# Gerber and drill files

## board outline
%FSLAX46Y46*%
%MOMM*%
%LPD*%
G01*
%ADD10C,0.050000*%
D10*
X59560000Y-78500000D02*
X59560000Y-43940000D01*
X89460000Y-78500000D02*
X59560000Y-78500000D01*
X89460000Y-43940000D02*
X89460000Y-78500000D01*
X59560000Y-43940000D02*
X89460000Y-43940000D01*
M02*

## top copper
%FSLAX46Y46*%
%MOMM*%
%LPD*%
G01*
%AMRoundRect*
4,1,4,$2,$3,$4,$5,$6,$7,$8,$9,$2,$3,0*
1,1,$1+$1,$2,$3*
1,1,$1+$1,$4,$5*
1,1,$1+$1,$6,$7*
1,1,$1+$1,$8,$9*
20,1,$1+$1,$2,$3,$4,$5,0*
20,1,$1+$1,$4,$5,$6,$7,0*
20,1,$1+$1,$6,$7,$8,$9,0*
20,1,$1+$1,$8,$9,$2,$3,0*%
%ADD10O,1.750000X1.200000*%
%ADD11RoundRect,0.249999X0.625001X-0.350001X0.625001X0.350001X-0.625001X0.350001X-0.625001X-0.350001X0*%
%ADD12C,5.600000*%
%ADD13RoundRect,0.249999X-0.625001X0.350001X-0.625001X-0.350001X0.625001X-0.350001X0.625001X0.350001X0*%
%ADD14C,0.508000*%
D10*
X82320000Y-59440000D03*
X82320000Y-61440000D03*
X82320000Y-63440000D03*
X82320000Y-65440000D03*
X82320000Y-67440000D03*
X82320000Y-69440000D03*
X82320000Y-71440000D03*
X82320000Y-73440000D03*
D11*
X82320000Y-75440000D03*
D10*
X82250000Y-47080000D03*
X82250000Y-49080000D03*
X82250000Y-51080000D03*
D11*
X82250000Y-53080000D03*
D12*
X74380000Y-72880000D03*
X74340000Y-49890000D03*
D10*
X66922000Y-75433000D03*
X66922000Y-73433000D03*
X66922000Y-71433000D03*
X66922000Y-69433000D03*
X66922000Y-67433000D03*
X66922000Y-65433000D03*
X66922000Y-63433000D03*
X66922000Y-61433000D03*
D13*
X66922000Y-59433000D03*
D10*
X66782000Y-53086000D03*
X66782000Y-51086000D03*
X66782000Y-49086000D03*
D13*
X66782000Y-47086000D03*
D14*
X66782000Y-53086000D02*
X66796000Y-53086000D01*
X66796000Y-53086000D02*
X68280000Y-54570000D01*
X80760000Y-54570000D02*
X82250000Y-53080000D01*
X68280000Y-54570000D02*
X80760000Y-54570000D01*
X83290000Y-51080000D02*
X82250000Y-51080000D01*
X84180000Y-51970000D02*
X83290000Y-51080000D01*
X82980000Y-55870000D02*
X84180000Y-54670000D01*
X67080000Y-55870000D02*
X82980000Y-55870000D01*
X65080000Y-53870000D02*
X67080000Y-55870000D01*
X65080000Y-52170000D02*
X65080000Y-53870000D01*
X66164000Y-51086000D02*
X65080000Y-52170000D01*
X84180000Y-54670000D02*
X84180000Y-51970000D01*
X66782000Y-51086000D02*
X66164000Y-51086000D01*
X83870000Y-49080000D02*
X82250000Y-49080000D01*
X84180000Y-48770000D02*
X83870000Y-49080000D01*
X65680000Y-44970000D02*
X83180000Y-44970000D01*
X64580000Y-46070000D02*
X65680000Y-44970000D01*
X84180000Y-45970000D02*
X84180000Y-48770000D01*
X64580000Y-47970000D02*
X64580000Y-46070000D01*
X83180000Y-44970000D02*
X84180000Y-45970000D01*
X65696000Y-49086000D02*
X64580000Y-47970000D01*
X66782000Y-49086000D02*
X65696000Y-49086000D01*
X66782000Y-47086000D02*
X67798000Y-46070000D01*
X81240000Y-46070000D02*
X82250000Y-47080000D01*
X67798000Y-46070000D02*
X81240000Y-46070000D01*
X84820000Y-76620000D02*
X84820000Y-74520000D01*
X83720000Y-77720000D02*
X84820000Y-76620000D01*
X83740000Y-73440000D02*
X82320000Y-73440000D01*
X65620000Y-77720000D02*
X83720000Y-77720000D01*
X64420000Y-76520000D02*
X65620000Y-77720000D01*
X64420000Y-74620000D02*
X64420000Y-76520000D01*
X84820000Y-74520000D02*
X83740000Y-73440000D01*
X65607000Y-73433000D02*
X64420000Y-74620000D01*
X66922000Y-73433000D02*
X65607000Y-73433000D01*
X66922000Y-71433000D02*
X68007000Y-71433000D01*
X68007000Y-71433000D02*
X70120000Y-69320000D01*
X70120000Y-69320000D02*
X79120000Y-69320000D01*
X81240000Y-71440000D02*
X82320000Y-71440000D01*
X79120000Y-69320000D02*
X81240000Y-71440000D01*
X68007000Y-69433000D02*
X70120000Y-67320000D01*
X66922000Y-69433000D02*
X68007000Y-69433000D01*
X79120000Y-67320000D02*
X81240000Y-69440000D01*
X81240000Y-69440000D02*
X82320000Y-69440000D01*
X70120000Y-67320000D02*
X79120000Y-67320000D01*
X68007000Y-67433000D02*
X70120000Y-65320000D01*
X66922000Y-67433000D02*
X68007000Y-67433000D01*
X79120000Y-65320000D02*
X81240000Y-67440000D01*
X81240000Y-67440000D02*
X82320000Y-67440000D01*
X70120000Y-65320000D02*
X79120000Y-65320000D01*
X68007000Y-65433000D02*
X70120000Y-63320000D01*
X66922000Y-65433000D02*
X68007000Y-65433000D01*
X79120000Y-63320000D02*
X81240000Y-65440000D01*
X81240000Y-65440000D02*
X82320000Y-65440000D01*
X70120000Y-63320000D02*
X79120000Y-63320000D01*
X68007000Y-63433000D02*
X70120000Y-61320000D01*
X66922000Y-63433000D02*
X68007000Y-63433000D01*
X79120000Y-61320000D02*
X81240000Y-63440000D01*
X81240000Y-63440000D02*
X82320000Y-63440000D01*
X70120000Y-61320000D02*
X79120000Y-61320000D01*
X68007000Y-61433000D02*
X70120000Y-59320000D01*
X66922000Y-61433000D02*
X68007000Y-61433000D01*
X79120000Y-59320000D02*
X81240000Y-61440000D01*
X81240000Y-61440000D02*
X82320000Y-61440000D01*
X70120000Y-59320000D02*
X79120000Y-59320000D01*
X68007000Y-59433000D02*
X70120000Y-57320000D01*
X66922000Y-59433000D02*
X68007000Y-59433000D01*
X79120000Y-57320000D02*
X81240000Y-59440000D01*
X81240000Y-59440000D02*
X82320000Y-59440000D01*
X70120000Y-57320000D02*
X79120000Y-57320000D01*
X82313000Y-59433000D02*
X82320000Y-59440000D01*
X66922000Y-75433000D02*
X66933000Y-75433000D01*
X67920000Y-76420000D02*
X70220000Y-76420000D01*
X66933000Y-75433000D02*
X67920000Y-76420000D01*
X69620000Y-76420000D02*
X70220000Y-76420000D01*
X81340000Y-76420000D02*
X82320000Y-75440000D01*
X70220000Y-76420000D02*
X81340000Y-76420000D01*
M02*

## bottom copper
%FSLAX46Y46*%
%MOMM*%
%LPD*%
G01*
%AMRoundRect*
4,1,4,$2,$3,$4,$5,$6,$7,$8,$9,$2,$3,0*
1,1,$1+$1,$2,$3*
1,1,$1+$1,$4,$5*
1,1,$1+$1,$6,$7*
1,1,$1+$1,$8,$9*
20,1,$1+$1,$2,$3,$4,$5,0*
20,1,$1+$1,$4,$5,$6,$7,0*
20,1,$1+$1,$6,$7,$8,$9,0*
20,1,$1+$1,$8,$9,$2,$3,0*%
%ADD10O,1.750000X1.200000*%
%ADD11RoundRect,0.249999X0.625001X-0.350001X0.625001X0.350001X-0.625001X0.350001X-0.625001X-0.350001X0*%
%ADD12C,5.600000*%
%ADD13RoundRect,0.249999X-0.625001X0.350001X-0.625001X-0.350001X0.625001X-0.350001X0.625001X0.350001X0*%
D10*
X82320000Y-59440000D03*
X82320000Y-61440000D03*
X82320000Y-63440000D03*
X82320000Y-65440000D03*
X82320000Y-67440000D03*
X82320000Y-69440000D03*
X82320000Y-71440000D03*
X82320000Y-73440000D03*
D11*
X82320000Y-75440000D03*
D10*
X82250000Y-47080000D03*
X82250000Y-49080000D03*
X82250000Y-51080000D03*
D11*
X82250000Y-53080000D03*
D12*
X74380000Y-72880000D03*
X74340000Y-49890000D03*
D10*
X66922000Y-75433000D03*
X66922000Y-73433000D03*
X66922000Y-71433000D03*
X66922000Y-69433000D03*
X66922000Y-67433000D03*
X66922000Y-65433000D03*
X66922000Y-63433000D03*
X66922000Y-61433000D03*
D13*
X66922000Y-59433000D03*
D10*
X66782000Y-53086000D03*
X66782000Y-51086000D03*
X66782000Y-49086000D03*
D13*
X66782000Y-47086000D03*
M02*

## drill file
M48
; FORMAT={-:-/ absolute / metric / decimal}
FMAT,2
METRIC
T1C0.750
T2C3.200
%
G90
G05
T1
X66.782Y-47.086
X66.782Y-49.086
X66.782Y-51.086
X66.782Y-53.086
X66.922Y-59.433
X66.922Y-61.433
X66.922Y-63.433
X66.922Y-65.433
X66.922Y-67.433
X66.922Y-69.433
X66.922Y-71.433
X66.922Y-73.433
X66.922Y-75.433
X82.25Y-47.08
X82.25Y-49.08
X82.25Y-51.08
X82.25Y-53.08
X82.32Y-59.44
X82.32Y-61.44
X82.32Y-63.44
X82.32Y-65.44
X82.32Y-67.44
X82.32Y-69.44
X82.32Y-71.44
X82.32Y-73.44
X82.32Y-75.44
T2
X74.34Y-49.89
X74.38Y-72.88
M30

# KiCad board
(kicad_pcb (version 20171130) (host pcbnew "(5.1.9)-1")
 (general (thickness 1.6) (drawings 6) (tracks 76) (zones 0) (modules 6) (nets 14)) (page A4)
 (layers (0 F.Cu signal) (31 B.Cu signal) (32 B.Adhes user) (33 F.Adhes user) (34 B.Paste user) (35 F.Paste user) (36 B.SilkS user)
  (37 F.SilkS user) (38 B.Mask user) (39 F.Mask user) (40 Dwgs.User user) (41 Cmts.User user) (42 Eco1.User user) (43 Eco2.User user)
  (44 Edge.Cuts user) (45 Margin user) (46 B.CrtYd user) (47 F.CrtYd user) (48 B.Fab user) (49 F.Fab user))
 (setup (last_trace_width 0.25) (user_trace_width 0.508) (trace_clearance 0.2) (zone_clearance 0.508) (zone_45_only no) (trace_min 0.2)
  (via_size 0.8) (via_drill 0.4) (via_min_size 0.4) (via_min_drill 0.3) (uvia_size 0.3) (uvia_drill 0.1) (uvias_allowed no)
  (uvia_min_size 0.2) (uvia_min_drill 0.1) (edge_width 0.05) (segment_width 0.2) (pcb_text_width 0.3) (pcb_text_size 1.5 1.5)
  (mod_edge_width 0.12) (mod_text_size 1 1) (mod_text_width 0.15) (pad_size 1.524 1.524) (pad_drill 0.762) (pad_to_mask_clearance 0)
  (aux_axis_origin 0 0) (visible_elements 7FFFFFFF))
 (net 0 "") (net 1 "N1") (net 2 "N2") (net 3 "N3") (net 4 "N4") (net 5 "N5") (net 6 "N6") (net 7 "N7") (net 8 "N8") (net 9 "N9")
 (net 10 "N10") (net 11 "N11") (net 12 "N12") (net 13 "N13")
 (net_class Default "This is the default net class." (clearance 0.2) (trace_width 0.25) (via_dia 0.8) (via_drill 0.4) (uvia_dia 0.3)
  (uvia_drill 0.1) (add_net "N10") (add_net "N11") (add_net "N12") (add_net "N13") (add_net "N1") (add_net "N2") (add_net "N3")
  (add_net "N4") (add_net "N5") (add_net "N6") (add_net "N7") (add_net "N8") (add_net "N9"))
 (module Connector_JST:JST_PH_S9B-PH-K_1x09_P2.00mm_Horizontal (layer F.Cu) (at 82.32 75.44 90)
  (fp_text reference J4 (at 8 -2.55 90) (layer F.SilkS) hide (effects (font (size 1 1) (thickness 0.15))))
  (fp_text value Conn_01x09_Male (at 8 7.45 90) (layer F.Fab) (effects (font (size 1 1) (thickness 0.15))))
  (pad 9 thru_hole oval (at 16 0 90) (size 1.2 1.75) (drill 0.75) (layers *.Cu *.Mask) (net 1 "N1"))
  (pad 8 thru_hole oval (at 14 0 90) (size 1.2 1.75) (drill 0.75) (layers *.Cu *.Mask) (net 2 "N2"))
  (pad 7 thru_hole oval (at 12 0 90) (size 1.2 1.75) (drill 0.75) (layers *.Cu *.Mask) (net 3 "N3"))
  (pad 6 thru_hole oval (at 10 0 90) (size 1.2 1.75) (drill 0.75) (layers *.Cu *.Mask) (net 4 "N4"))
  (pad 5 thru_hole oval (at 8 0 90) (size 1.2 1.75) (drill 0.75) (layers *.Cu *.Mask) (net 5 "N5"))
  (pad 4 thru_hole oval (at 6 0 90) (size 1.2 1.75) (drill 0.75) (layers *.Cu *.Mask) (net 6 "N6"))
  (pad 3 thru_hole oval (at 4 0 90) (size 1.2 1.75) (drill 0.75) (layers *.Cu *.Mask) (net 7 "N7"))
  (pad 2 thru_hole oval (at 2 0 90) (size 1.2 1.75) (drill 0.75) (layers *.Cu *.Mask) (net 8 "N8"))
  (pad 1 thru_hole roundrect (at 0 0 90) (size 1.2 1.75) (drill 0.75) (layers *.Cu *.Mask) (roundrect_rratio 0.2083325) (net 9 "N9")))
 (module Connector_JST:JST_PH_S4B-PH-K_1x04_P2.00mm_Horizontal (layer F.Cu) (at 82.25 53.08 90)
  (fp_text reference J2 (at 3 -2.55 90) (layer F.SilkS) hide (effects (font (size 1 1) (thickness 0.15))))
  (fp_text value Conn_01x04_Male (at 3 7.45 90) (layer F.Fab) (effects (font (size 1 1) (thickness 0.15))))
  (pad 4 thru_hole oval (at 6 0 90) (size 1.2 1.75) (drill 0.75) (layers *.Cu *.Mask) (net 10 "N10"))
  (pad 3 thru_hole oval (at 4 0 90) (size 1.2 1.75) (drill 0.75) (layers *.Cu *.Mask) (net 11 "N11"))
  (pad 2 thru_hole oval (at 2 0 90) (size 1.2 1.75) (drill 0.75) (layers *.Cu *.Mask) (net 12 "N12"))
  (pad 1 thru_hole roundrect (at 0 0 90) (size 1.2 1.75) (drill 0.75) (layers *.Cu *.Mask) (roundrect_rratio 0.2083325) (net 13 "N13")))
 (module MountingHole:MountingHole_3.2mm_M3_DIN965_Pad (layer F.Cu) (at 74.38 72.88)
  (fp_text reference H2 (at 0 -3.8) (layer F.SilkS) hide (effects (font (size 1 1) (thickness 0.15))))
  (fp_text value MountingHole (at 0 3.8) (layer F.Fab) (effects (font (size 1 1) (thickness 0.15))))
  (pad 1 thru_hole circle (at 0 0) (size 5.6 5.6) (drill 3.2) (layers *.Cu *.Mask)))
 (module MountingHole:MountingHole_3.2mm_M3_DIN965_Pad (layer F.Cu) (at 74.34 49.89)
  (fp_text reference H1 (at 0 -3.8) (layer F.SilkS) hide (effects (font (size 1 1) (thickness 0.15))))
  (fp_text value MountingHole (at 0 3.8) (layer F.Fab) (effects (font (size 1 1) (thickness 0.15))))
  (pad 1 thru_hole circle (at 0 0) (size 5.6 5.6) (drill 3.2) (layers *.Cu *.Mask)))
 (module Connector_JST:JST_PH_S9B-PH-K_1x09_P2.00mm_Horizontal (layer F.Cu) (at 66.922 59.433 270)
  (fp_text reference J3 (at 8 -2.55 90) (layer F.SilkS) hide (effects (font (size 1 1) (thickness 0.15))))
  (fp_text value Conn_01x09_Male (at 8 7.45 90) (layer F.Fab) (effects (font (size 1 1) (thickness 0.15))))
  (pad 9 thru_hole oval (at 16 0 270) (size 1.2 1.75) (drill 0.75) (layers *.Cu *.Mask) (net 9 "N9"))
  (pad 8 thru_hole oval (at 14 0 270) (size 1.2 1.75) (drill 0.75) (layers *.Cu *.Mask) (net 8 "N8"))
  (pad 7 thru_hole oval (at 12 0 270) (size 1.2 1.75) (drill 0.75) (layers *.Cu *.Mask) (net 7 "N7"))
  (pad 6 thru_hole oval (at 10 0 270) (size 1.2 1.75) (drill 0.75) (layers *.Cu *.Mask) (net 6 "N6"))
  (pad 5 thru_hole oval (at 8 0 270) (size 1.2 1.75) (drill 0.75) (layers *.Cu *.Mask) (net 5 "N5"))
  (pad 4 thru_hole oval (at 6 0 270) (size 1.2 1.75) (drill 0.75) (layers *.Cu *.Mask) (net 4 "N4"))
  (pad 3 thru_hole oval (at 4 0 270) (size 1.2 1.75) (drill 0.75) (layers *.Cu *.Mask) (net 3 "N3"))
  (pad 2 thru_hole oval (at 2 0 270) (size 1.2 1.75) (drill 0.75) (layers *.Cu *.Mask) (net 2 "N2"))
  (pad 1 thru_hole roundrect (at 0 0 270) (size 1.2 1.75) (drill 0.75) (layers *.Cu *.Mask) (roundrect_rratio 0.2083325) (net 1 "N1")))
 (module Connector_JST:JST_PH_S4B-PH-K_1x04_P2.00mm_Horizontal (layer F.Cu) (at 66.782 47.086 270)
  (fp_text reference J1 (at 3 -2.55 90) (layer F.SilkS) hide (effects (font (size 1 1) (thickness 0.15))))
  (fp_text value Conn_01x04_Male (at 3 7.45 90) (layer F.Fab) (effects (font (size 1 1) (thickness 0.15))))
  (pad 4 thru_hole oval (at 6 0 270) (size 1.2 1.75) (drill 0.75) (layers *.Cu *.Mask) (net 13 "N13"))
  (pad 3 thru_hole oval (at 4 0 270) (size 1.2 1.75) (drill 0.75) (layers *.Cu *.Mask) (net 12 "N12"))
  (pad 2 thru_hole oval (at 2 0 270) (size 1.2 1.75) (drill 0.75) (layers *.Cu *.Mask) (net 11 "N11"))
  (pad 1 thru_hole roundrect (at 0 0 270) (size 1.2 1.75) (drill 0.75) (layers *.Cu *.Mask) (roundrect_rratio 0.2083325) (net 10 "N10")))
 (gr_line (start 59.56 78.5) (end 59.56 43.94) (layer Edge.Cuts) (width 0.05))
 (gr_line (start 89.46 78.5) (end 59.56 78.5) (layer Edge.Cuts) (width 0.05))
 (gr_line (start 89.46 43.94) (end 89.46 78.5) (layer Edge.Cuts) (width 0.05))
 (gr_line (start 59.56 43.94) (end 89.46 43.94) (layer Edge.Cuts) (width 0.05))
 (segment (start 66.782 53.086) (end 66.796 53.086) (width 0.508) (layer F.Cu) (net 13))
 (segment (start 66.796 53.086) (end 68.28 54.57) (width 0.508) (layer F.Cu) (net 13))
 (segment (start 80.76 54.57) (end 82.25 53.08) (width 0.508) (layer F.Cu) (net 13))
 (segment (start 68.28 54.57) (end 80.76 54.57) (width 0.508) (layer F.Cu) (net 13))
 (segment (start 83.29 51.08) (end 82.25 51.08) (width 0.508) (layer F.Cu) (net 12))
 (segment (start 84.18 51.97) (end 83.29 51.08) (width 0.508) (layer F.Cu) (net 12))
 (segment (start 82.98 55.87) (end 84.18 54.67) (width 0.508) (layer F.Cu) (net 12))
 (segment (start 67.08 55.87) (end 82.98 55.87) (width 0.508) (layer F.Cu) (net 12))
 (segment (start 65.08 53.87) (end 67.08 55.87) (width 0.508) (layer F.Cu) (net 12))
 (segment (start 65.08 52.17) (end 65.08 53.87) (width 0.508) (layer F.Cu) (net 12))
 (segment (start 66.164 51.086) (end 65.08 52.17) (width 0.508) (layer F.Cu) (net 12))
 (segment (start 84.18 54.67) (end 84.18 51.97) (width 0.508) (layer F.Cu) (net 12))
 (segment (start 66.782 51.086) (end 66.164 51.086) (width 0.508) (layer F.Cu) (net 12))
 (segment (start 83.87 49.08) (end 82.25 49.08) (width 0.508) (layer F.Cu) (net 11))
 (segment (start 84.18 48.77) (end 83.87 49.08) (width 0.508) (layer F.Cu) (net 11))
 (segment (start 65.68 44.97) (end 83.18 44.97) (width 0.508) (layer F.Cu) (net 11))
 (segment (start 64.58 46.07) (end 65.68 44.97) (width 0.508) (layer F.Cu) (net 11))
 (segment (start 84.18 45.97) (end 84.18 48.77) (width 0.508) (layer F.Cu) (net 11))
 (segment (start 64.58 47.97) (end 64.58 46.07) (width 0.508) (layer F.Cu) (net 11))
 (segment (start 83.18 44.97) (end 84.18 45.97) (width 0.508) (layer F.Cu) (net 11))
 (segment (start 65.696 49.086) (end 64.58 47.97) (width 0.508) (layer F.Cu) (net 11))
 (segment (start 66.782 49.086) (end 65.696 49.086) (width 0.508) (layer F.Cu) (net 11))
 (segment (start 66.782 47.086) (end 67.798 46.07) (width 0.508) (layer F.Cu) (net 10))
 (segment (start 81.24 46.07) (end 82.25 47.08) (width 0.508) (layer F.Cu) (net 10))
 (segment (start 67.798 46.07) (end 81.24 46.07) (width 0.508) (layer F.Cu) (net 10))
 (segment (start 84.82 76.62) (end 84.82 74.52) (width 0.508) (layer F.Cu) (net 8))
 (segment (start 83.72 77.72) (end 84.82 76.62) (width 0.508) (layer F.Cu) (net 8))
 (segment (start 83.74 73.44) (end 82.32 73.44) (width 0.508) (layer F.Cu) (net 8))
 (segment (start 65.62 77.72) (end 83.72 77.72) (width 0.508) (layer F.Cu) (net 8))
 (segment (start 64.42 76.52) (end 65.62 77.72) (width 0.508) (layer F.Cu) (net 8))
 (segment (start 64.42 74.62) (end 64.42 76.52) (width 0.508) (layer F.Cu) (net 8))
 (segment (start 84.82 74.52) (end 83.74 73.44) (width 0.508) (layer F.Cu) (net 8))
 (segment (start 65.607 73.433) (end 64.42 74.62) (width 0.508) (layer F.Cu) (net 8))
 (segment (start 66.922 73.433) (end 65.607 73.433) (width 0.508) (layer F.Cu) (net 8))
 (segment (start 66.922 71.433) (end 68.007 71.433) (width 0.508) (layer F.Cu) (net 7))
 (segment (start 68.007 71.433) (end 70.12 69.32) (width 0.508) (layer F.Cu) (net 7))
 (segment (start 70.12 69.32) (end 79.12 69.32) (width 0.508) (layer F.Cu) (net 7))
 (segment (start 81.24 71.44) (end 82.32 71.44) (width 0.508) (layer F.Cu) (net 7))
 (segment (start 79.12 69.32) (end 81.24 71.44) (width 0.508) (layer F.Cu) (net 7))
 (segment (start 68.007 69.433) (end 70.12 67.32) (width 0.508) (layer F.Cu) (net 6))
 (segment (start 66.922 69.433) (end 68.007 69.433) (width 0.508) (layer F.Cu) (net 6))
 (segment (start 79.12 67.32) (end 81.24 69.44) (width 0.508) (layer F.Cu) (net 6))
 (segment (start 81.24 69.44) (end 82.32 69.44) (width 0.508) (layer F.Cu) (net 6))
 (segment (start 70.12 67.32) (end 79.12 67.32) (width 0.508) (layer F.Cu) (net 6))
 (segment (start 68.007 67.433) (end 70.12 65.32) (width 0.508) (layer F.Cu) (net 5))
 (segment (start 66.922 67.433) (end 68.007 67.433) (width 0.508) (layer F.Cu) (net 5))
 (segment (start 79.12 65.32) (end 81.24 67.44) (width 0.508) (layer F.Cu) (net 5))
 (segment (start 81.24 67.44) (end 82.32 67.44) (width 0.508) (layer F.Cu) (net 5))
 (segment (start 70.12 65.32) (end 79.12 65.32) (width 0.508) (layer F.Cu) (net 5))
 (segment (start 68.007 65.433) (end 70.12 63.32) (width 0.508) (layer F.Cu) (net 4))
 (segment (start 66.922 65.433) (end 68.007 65.433) (width 0.508) (layer F.Cu) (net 4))
 (segment (start 79.12 63.32) (end 81.24 65.44) (width 0.508) (layer F.Cu) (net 4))
 (segment (start 81.24 65.44) (end 82.32 65.44) (width 0.508) (layer F.Cu) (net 4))
 (segment (start 70.12 63.32) (end 79.12 63.32) (width 0.508) (layer F.Cu) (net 4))
 (segment (start 68.007 63.433) (end 70.12 61.32) (width 0.508) (layer F.Cu) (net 3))
 (segment (start 66.922 63.433) (end 68.007 63.433) (width 0.508) (layer F.Cu) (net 3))
 (segment (start 79.12 61.32) (end 81.24 63.44) (width 0.508) (layer F.Cu) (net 3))
 (segment (start 81.24 63.44) (end 82.32 63.44) (width 0.508) (layer F.Cu) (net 3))
 (segment (start 70.12 61.32) (end 79.12 61.32) (width 0.508) (layer F.Cu) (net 3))
 (segment (start 68.007 61.433) (end 70.12 59.32) (width 0.508) (layer F.Cu) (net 2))
 (segment (start 66.922 61.433) (end 68.007 61.433) (width 0.508) (layer F.Cu) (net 2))
 (segment (start 79.12 59.32) (end 81.24 61.44) (width 0.508) (layer F.Cu) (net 2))
 (segment (start 81.24 61.44) (end 82.32 61.44) (width 0.508) (layer F.Cu) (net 2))
 (segment (start 70.12 59.32) (end 79.12 59.32) (width 0.508) (layer F.Cu) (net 2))
 (segment (start 68.007 59.433) (end 70.12 57.32) (width 0.508) (layer F.Cu) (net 1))
 (segment (start 66.922 59.433) (end 68.007 59.433) (width 0.508) (layer F.Cu) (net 1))
 (segment (start 79.12 57.32) (end 81.24 59.44) (width 0.508) (layer F.Cu) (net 1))
 (segment (start 81.24 59.44) (end 82.32 59.44) (width 0.508) (layer F.Cu) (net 1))
 (segment (start 70.12 57.32) (end 79.12 57.32) (width 0.508) (layer F.Cu) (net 1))
 (segment (start 82.313 59.433) (end 82.32 59.44) (width 0.508) (layer F.Cu) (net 1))
 (segment (start 66.922 75.433) (end 66.933 75.433) (width 0.508) (layer F.Cu) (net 9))
 (segment (start 67.92 76.42) (end 70.22 76.42) (width 0.508) (layer F.Cu) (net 9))
 (segment (start 66.933 75.433) (end 67.92 76.42) (width 0.508) (layer F.Cu) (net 9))
 (segment (start 69.62 76.42) (end 70.22 76.42) (width 0.508) (layer F.Cu) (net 9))
 (segment (start 81.34 76.42) (end 82.32 75.44) (width 0.508) (layer F.Cu) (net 9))
 (segment (start 70.22 76.42) (end 81.34 76.42) (width 0.508) (layer F.Cu) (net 9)))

